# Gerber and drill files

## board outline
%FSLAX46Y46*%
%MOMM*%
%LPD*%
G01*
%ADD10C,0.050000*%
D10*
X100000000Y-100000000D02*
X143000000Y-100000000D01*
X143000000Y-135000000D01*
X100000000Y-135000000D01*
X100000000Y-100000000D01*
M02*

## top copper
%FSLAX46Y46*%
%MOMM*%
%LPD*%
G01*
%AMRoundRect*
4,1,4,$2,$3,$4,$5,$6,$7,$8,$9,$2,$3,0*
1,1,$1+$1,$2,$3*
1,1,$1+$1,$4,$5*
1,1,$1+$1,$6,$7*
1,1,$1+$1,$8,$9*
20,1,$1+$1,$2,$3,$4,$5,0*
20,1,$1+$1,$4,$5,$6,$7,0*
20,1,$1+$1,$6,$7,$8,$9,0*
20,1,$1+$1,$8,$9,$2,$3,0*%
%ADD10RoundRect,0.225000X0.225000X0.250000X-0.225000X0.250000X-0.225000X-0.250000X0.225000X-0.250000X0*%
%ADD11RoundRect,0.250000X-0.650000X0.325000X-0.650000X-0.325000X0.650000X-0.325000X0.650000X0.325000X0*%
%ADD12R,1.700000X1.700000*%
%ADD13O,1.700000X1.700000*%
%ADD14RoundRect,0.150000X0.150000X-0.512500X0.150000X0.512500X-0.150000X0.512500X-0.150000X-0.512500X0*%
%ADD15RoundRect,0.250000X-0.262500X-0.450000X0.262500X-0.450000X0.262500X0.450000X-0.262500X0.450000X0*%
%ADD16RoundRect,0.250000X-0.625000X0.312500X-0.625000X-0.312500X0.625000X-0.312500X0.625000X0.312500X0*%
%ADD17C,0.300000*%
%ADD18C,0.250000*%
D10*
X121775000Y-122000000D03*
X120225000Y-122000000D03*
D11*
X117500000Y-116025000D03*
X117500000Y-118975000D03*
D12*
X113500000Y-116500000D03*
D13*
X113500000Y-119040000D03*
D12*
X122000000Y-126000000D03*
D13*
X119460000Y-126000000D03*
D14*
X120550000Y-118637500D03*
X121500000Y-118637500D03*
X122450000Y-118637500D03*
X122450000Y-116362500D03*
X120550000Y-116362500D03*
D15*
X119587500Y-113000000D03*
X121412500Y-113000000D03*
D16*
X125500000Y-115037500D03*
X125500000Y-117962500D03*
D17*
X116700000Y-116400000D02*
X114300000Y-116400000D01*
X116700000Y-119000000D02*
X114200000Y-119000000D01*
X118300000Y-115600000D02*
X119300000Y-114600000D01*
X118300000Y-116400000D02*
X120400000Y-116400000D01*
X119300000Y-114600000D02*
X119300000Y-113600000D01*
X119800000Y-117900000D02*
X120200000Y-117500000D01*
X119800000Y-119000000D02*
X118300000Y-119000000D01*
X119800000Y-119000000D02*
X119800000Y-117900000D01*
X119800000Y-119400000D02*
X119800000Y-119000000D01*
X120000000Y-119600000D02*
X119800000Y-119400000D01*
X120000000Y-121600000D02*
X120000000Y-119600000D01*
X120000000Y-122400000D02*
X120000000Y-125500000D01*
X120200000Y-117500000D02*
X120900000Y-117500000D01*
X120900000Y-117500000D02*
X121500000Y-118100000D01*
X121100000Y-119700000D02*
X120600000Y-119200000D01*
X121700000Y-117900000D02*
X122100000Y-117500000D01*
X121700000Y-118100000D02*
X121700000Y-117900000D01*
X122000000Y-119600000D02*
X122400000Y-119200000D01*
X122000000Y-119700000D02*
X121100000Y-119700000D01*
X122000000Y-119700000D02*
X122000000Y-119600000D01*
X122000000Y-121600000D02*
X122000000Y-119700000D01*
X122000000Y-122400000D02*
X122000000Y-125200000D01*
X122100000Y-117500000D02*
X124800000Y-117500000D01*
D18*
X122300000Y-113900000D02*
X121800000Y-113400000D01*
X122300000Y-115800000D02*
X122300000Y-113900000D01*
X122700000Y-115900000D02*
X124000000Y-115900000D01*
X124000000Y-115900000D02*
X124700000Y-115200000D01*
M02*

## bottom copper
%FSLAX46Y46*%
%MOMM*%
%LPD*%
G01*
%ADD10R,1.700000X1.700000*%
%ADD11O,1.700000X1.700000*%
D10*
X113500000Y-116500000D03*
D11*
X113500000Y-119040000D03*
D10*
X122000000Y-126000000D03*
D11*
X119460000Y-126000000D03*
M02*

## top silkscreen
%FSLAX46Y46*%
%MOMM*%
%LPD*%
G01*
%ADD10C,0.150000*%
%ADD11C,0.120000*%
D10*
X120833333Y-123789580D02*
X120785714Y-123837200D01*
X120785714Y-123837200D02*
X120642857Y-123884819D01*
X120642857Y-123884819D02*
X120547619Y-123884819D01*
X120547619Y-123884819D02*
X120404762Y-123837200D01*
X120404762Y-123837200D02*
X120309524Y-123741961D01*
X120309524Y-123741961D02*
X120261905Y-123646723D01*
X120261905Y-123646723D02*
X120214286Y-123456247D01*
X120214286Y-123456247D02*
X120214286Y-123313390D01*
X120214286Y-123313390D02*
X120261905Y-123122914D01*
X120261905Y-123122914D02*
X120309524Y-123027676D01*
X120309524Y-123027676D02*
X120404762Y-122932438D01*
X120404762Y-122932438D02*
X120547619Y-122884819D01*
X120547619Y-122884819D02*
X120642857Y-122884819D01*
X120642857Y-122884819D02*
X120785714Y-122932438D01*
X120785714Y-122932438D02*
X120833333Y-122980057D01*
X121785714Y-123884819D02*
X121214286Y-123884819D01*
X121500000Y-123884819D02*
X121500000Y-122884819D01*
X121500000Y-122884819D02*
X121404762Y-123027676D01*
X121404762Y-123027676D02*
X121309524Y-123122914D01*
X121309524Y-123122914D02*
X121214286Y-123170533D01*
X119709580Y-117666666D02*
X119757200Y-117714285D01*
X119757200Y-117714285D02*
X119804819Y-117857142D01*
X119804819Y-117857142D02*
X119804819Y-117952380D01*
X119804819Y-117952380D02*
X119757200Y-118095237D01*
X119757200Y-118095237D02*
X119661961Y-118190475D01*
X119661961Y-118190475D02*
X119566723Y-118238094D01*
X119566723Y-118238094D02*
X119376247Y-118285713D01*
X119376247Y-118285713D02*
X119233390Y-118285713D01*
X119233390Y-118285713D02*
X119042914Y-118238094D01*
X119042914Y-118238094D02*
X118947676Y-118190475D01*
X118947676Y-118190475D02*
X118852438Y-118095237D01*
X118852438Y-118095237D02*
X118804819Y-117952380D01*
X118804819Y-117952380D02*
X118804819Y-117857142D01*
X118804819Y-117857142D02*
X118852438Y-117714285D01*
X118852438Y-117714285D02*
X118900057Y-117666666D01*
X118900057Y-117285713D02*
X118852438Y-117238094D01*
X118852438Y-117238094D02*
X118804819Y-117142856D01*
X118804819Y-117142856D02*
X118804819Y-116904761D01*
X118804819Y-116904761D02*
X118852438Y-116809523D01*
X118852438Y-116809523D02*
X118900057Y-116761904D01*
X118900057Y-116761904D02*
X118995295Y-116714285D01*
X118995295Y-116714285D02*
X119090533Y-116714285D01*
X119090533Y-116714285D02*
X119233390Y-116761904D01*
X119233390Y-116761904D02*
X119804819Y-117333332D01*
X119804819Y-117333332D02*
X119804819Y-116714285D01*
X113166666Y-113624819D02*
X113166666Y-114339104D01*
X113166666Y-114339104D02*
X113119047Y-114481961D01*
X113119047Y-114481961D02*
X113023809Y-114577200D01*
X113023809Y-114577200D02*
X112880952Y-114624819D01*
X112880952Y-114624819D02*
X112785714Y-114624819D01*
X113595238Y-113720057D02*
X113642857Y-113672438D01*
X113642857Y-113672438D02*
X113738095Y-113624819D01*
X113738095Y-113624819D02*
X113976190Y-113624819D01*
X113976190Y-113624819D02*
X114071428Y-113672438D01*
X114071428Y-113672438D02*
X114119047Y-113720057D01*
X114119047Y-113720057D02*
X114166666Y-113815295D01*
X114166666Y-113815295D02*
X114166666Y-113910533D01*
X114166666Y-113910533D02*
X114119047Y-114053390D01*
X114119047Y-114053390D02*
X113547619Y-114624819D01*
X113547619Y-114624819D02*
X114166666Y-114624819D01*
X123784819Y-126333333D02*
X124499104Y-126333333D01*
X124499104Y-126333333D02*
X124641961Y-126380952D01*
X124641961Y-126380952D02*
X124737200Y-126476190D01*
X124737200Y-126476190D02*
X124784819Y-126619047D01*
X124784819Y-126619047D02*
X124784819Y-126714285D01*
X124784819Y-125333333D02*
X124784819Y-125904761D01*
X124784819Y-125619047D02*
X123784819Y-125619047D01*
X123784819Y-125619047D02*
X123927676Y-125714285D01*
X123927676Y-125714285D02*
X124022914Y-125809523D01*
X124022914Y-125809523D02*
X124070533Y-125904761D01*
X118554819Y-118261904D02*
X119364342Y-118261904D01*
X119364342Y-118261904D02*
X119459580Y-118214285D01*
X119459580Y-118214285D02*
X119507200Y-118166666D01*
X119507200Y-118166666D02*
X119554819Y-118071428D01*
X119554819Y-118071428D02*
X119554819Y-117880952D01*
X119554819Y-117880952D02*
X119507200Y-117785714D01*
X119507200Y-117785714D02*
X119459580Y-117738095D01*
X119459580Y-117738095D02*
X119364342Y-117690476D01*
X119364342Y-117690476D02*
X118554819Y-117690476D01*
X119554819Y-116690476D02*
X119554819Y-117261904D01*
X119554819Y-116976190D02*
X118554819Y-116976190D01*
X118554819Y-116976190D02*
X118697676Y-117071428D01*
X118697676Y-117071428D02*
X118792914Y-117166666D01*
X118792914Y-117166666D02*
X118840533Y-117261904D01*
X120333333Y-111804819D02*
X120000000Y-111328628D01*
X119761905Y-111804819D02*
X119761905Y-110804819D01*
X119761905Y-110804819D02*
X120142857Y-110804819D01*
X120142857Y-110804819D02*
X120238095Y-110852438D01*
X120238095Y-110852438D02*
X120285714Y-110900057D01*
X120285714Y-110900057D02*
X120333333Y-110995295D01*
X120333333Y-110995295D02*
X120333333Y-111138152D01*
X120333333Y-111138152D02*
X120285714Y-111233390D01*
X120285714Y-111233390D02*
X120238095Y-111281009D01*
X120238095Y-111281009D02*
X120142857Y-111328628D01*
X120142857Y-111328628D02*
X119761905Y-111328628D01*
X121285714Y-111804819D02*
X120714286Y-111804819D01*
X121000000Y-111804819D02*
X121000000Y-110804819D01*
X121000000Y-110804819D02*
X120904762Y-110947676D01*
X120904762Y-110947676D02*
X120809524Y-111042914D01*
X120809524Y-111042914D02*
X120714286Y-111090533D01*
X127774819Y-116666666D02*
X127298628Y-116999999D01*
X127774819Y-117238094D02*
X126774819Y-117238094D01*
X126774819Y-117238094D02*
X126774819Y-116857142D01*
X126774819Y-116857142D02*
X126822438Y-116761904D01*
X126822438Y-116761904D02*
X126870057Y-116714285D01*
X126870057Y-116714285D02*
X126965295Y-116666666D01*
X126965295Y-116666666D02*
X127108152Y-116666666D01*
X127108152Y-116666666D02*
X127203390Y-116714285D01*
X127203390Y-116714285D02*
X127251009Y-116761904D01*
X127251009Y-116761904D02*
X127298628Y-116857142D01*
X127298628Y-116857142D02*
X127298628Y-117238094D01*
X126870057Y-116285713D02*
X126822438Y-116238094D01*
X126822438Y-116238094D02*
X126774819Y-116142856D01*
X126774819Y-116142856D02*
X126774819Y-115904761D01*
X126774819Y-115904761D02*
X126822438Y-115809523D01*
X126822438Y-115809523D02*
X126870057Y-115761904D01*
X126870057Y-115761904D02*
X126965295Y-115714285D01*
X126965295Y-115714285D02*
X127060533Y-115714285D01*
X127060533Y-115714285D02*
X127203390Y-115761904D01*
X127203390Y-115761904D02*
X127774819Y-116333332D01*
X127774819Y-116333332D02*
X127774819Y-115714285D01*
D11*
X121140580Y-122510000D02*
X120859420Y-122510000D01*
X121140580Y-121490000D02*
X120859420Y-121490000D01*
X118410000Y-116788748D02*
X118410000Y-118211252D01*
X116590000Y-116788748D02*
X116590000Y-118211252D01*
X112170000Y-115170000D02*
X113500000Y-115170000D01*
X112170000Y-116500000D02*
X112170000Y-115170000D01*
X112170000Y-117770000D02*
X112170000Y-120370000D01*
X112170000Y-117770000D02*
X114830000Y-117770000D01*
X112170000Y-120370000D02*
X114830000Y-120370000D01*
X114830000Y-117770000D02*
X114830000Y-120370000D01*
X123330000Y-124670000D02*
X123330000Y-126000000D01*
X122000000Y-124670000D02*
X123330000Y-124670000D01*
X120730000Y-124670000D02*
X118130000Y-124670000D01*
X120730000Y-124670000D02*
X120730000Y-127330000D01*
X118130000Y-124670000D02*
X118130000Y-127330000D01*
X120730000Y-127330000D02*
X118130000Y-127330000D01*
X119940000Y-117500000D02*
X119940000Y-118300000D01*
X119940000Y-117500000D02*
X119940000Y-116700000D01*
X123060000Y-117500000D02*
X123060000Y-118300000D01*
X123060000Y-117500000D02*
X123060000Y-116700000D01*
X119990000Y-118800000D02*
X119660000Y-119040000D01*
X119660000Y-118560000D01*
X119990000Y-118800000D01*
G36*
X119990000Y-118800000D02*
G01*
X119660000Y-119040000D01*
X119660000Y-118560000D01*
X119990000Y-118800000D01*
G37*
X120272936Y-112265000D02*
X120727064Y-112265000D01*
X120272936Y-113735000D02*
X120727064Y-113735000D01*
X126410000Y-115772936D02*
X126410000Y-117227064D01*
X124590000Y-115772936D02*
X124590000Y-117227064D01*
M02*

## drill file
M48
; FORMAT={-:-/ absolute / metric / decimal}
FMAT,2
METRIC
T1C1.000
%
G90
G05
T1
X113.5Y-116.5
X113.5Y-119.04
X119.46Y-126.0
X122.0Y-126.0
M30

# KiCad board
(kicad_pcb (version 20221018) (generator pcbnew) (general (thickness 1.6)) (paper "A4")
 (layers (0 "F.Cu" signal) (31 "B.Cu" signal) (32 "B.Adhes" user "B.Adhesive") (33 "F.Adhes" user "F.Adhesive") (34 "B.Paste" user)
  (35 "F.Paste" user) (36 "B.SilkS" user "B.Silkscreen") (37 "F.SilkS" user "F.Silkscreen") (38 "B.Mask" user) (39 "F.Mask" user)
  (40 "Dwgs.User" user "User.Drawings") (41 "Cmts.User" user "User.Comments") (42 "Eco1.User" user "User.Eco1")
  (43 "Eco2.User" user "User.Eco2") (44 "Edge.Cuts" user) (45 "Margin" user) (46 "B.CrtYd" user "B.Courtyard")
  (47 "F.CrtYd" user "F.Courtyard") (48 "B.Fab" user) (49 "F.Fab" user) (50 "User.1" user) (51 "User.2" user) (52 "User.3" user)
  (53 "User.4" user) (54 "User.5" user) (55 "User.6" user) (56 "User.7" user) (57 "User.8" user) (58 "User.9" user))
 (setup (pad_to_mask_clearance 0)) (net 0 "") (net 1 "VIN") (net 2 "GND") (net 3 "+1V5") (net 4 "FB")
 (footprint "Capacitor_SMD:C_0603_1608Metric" (layer "F.Cu") (at 121 122 180)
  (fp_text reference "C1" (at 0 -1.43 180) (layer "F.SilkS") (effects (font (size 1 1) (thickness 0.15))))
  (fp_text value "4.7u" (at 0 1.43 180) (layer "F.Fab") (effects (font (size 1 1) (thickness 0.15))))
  (fp_line (start -0.14058 -0.51) (end 0.14058 -0.51) (stroke (width 0.12) (type solid)) (layer "F.SilkS"))
  (fp_line (start -0.14058 0.51) (end 0.14058 0.51) (stroke (width 0.12) (type solid)) (layer "F.SilkS"))
  (pad "1" smd roundrect (at -0.775 0 180) (size 0.9 0.95) (layers "F.Cu" "F.Paste" "F.Mask") (roundrect_rratio 0.25) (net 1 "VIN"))
  (pad "2" smd roundrect (at 0.775 0 180) (size 0.9 0.95) (layers "F.Cu" "F.Paste" "F.Mask") (roundrect_rratio 0.25) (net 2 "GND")))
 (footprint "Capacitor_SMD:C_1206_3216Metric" (layer "F.Cu") (at 117.5 117.5 -90)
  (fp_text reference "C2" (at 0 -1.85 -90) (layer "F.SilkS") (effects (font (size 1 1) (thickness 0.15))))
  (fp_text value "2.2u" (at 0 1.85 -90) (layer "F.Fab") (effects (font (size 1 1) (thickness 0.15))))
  (fp_line (start -0.711252 -0.91) (end 0.711252 -0.91) (stroke (width 0.12) (type solid)) (layer "F.SilkS"))
  (fp_line (start -0.711252 0.91) (end 0.711252 0.91) (stroke (width 0.12) (type solid)) (layer "F.SilkS"))
  (pad "1" smd roundrect (at -1.475 0 270) (size 1.15 1.8) (layers "F.Cu" "F.Paste" "F.Mask") (roundrect_rratio 0.217391) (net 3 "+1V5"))
  (pad "2" smd roundrect (at 1.475 0 270) (size 1.15 1.8) (layers "F.Cu" "F.Paste" "F.Mask") (roundrect_rratio 0.217391) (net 2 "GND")))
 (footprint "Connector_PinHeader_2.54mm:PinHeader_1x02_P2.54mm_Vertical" (layer "F.Cu") (at 113.5 116.5)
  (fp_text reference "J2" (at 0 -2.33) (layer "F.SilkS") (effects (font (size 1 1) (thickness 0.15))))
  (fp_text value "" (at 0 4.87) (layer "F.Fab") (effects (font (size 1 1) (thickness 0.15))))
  (fp_line (start -1.33 -1.33) (end 0 -1.33) (stroke (width 0.12) (type solid)) (layer "F.SilkS"))
  (fp_line (start -1.33 0) (end -1.33 -1.33) (stroke (width 0.12) (type solid)) (layer "F.SilkS"))
  (fp_line (start -1.33 1.27) (end -1.33 3.87) (stroke (width 0.12) (type solid)) (layer "F.SilkS"))
  (fp_line (start -1.33 1.27) (end 1.33 1.27) (stroke (width 0.12) (type solid)) (layer "F.SilkS"))
  (fp_line (start -1.33 3.87) (end 1.33 3.87) (stroke (width 0.12) (type solid)) (layer "F.SilkS"))
  (fp_line (start 1.33 1.27) (end 1.33 3.87) (stroke (width 0.12) (type solid)) (layer "F.SilkS"))
  (pad "1" thru_hole rect (at 0 0) (size 1.7 1.7) (drill 1) (layers "*.Cu" "*.Mask") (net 3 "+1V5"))
  (pad "2" thru_hole oval (at 0 2.54) (size 1.7 1.7) (drill 1) (layers "*.Cu" "*.Mask") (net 2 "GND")))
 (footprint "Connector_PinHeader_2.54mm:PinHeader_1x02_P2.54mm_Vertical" (layer "F.Cu") (at 122 126 -90)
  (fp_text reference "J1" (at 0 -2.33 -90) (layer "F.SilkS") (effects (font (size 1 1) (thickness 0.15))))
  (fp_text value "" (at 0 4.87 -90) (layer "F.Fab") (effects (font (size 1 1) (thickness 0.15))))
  (fp_line (start -1.33 -1.33) (end 0 -1.33) (stroke (width 0.12) (type solid)) (layer "F.SilkS"))
  (fp_line (start -1.33 0) (end -1.33 -1.33) (stroke (width 0.12) (type solid)) (layer "F.SilkS"))
  (fp_line (start -1.33 1.27) (end -1.33 3.87) (stroke (width 0.12) (type solid)) (layer "F.SilkS"))
  (fp_line (start -1.33 1.27) (end 1.33 1.27) (stroke (width 0.12) (type solid)) (layer "F.SilkS"))
  (fp_line (start -1.33 3.87) (end 1.33 3.87) (stroke (width 0.12) (type solid)) (layer "F.SilkS"))
  (fp_line (start 1.33 1.27) (end 1.33 3.87) (stroke (width 0.12) (type solid)) (layer "F.SilkS"))
  (pad "1" thru_hole rect (at 0 0 270) (size 1.7 1.7) (drill 1) (layers "*.Cu" "*.Mask") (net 1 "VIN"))
  (pad "2" thru_hole oval (at 0 2.54 270) (size 1.7 1.7) (drill 1) (layers "*.Cu" "*.Mask") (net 2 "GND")))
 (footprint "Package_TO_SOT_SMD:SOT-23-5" (layer "F.Cu") (at 121.5 117.5 90)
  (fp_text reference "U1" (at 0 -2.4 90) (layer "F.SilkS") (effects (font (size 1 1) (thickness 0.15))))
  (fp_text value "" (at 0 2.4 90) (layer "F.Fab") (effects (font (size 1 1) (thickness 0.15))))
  (fp_line (start 0 -1.56) (end -0.8 -1.56) (stroke (width 0.12) (type solid)) (layer "F.SilkS"))
  (fp_line (start 0 -1.56) (end 0.8 -1.56) (stroke (width 0.12) (type solid)) (layer "F.SilkS"))
  (fp_line (start 0 1.56) (end -0.8 1.56) (stroke (width 0.12) (type solid)) (layer "F.SilkS"))
  (fp_line (start 0 1.56) (end 0.8 1.56) (stroke (width 0.12) (type solid)) (layer "F.SilkS"))
  (fp_poly
   (pts (xy -1.3 -1.51) (xy -1.54 -1.84) (xy -1.06 -1.84) (xy -1.3 -1.51)) (stroke (width 0.12) (type solid)) (fill solid) (layer "F.SilkS"))
  (pad "1" smd roundrect (at -1.1375 -0.95 90) (size 1.325 0.6) (layers "F.Cu" "F.Paste" "F.Mask") (roundrect_rratio 0.25) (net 1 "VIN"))
  (pad "2" smd roundrect (at -1.1375 0 90) (size 1.325 0.6) (layers "F.Cu" "F.Paste" "F.Mask") (roundrect_rratio 0.25) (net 2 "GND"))
  (pad "3" smd roundrect (at -1.1375 0.95 90) (size 1.325 0.6) (layers "F.Cu" "F.Paste" "F.Mask") (roundrect_rratio 0.25) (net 1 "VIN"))
  (pad "4" smd roundrect (at 1.1375 0.95 90) (size 1.325 0.6) (layers "F.Cu" "F.Paste" "F.Mask") (roundrect_rratio 0.25) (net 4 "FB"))
  (pad "5" smd roundrect (at 1.1375 -0.95 90) (size 1.325 0.6) (layers "F.Cu" "F.Paste" "F.Mask") (roundrect_rratio 0.25) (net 3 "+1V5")))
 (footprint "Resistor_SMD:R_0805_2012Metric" (layer "F.Cu") (at 120.5 113)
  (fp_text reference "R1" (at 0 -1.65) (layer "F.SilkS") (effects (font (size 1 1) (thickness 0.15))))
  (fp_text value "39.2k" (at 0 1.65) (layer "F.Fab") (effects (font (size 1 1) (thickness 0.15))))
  (fp_line (start -0.227064 -0.735) (end 0.227064 -0.735) (stroke (width 0.12) (type solid)) (layer "F.SilkS"))
  (fp_line (start -0.227064 0.735) (end 0.227064 0.735) (stroke (width 0.12) (type solid)) (layer "F.SilkS"))
  (pad "1" smd roundrect (at -0.9125 0) (size 1.025 1.4) (layers "F.Cu" "F.Paste" "F.Mask") (roundrect_rratio 0.243902) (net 3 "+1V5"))
  (pad "2" smd roundrect (at 0.9125 0) (size 1.025 1.4) (layers "F.Cu" "F.Paste" "F.Mask") (roundrect_rratio 0.243902) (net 4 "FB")))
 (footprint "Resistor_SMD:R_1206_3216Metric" (layer "F.Cu") (at 125.5 116.5 -90)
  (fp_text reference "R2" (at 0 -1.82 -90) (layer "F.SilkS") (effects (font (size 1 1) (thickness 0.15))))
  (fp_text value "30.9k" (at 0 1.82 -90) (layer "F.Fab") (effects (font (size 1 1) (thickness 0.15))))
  (fp_line (start -0.727064 -0.91) (end 0.727064 -0.91) (stroke (width 0.12) (type solid)) (layer "F.SilkS"))
  (fp_line (start -0.727064 0.91) (end 0.727064 0.91) (stroke (width 0.12) (type solid)) (layer "F.SilkS"))
  (pad "1" smd roundrect (at -1.4625 0 270) (size 1.125 1.75) (layers "F.Cu" "F.Paste" "F.Mask") (roundrect_rratio 0.222222) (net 4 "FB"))
  (pad "2" smd roundrect (at 1.4625 0 270) (size 1.125 1.75) (layers "F.Cu" "F.Paste" "F.Mask") (roundrect_rratio 0.222222) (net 2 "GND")))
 (gr_rect (start 100 100) (end 143 135) (stroke (width 0.05) (type default)) (fill none) (layer "Edge.Cuts"))
 (segment (start 116.7 116.4) (end 114.3 116.4) (width 0.3) (layer "F.Cu") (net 3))
 (segment (start 116.7 119) (end 114.2 119) (width 0.3) (layer "F.Cu") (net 2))
 (segment (start 118.3 115.6) (end 119.3 114.6) (width 0.3) (layer "F.Cu") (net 3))
 (segment (start 118.3 116.4) (end 120.4 116.4) (width 0.3) (layer "F.Cu") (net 3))
 (segment (start 119.3 114.6) (end 119.3 113.6) (width 0.3) (layer "F.Cu") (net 3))
 (segment (start 119.8 117.9) (end 120.2 117.5) (width 0.3) (layer "F.Cu") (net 2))
 (segment (start 119.8 119) (end 118.3 119) (width 0.3) (layer "F.Cu") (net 2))
 (segment (start 119.8 119) (end 119.8 117.9) (width 0.3) (layer "F.Cu") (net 2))
 (segment (start 119.8 119.4) (end 119.8 119) (width 0.3) (layer "F.Cu") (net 2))
 (segment (start 120 119.6) (end 119.8 119.4) (width 0.3) (layer "F.Cu") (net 2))
 (segment (start 120 121.6) (end 120 119.6) (width 0.3) (layer "F.Cu") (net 2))
 (segment (start 120 122.4) (end 120 125.5) (width 0.3) (layer "F.Cu") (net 2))
 (segment (start 120.2 117.5) (end 120.9 117.5) (width 0.3) (layer "F.Cu") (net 2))
 (segment (start 120.9 117.5) (end 121.5 118.1) (width 0.3) (layer "F.Cu") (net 2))
 (segment (start 121.1 119.7) (end 120.6 119.2) (width 0.3) (layer "F.Cu") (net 1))
 (segment (start 121.7 117.9) (end 122.1 117.5) (width 0.3) (layer "F.Cu") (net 2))
 (segment (start 121.7 118.1) (end 121.7 117.9) (width 0.3) (layer "F.Cu") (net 2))
 (segment (start 122 119.6) (end 122.4 119.2) (width 0.3) (layer "F.Cu") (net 1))
 (segment (start 122 119.7) (end 121.1 119.7) (width 0.3) (layer "F.Cu") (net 1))
 (segment (start 122 119.7) (end 122 119.6) (width 0.3) (layer "F.Cu") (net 1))
 (segment (start 122 121.6) (end 122 119.7) (width 0.3) (layer "F.Cu") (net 1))
 (segment (start 122 122.4) (end 122 125.2) (width 0.3) (layer "F.Cu") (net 1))
 (segment (start 122.1 117.5) (end 124.8 117.5) (width 0.3) (layer "F.Cu") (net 2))
 (segment (start 122.3 113.9) (end 121.8 113.4) (width 0.25) (layer "F.Cu") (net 4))
 (segment (start 122.3 115.8) (end 122.3 113.9) (width 0.25) (layer "F.Cu") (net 4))
 (segment (start 122.7 115.9) (end 124 115.9) (width 0.25) (layer "F.Cu") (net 4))
 (segment (start 124 115.9) (end 124.7 115.2) (width 0.25) (layer "F.Cu") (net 4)))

